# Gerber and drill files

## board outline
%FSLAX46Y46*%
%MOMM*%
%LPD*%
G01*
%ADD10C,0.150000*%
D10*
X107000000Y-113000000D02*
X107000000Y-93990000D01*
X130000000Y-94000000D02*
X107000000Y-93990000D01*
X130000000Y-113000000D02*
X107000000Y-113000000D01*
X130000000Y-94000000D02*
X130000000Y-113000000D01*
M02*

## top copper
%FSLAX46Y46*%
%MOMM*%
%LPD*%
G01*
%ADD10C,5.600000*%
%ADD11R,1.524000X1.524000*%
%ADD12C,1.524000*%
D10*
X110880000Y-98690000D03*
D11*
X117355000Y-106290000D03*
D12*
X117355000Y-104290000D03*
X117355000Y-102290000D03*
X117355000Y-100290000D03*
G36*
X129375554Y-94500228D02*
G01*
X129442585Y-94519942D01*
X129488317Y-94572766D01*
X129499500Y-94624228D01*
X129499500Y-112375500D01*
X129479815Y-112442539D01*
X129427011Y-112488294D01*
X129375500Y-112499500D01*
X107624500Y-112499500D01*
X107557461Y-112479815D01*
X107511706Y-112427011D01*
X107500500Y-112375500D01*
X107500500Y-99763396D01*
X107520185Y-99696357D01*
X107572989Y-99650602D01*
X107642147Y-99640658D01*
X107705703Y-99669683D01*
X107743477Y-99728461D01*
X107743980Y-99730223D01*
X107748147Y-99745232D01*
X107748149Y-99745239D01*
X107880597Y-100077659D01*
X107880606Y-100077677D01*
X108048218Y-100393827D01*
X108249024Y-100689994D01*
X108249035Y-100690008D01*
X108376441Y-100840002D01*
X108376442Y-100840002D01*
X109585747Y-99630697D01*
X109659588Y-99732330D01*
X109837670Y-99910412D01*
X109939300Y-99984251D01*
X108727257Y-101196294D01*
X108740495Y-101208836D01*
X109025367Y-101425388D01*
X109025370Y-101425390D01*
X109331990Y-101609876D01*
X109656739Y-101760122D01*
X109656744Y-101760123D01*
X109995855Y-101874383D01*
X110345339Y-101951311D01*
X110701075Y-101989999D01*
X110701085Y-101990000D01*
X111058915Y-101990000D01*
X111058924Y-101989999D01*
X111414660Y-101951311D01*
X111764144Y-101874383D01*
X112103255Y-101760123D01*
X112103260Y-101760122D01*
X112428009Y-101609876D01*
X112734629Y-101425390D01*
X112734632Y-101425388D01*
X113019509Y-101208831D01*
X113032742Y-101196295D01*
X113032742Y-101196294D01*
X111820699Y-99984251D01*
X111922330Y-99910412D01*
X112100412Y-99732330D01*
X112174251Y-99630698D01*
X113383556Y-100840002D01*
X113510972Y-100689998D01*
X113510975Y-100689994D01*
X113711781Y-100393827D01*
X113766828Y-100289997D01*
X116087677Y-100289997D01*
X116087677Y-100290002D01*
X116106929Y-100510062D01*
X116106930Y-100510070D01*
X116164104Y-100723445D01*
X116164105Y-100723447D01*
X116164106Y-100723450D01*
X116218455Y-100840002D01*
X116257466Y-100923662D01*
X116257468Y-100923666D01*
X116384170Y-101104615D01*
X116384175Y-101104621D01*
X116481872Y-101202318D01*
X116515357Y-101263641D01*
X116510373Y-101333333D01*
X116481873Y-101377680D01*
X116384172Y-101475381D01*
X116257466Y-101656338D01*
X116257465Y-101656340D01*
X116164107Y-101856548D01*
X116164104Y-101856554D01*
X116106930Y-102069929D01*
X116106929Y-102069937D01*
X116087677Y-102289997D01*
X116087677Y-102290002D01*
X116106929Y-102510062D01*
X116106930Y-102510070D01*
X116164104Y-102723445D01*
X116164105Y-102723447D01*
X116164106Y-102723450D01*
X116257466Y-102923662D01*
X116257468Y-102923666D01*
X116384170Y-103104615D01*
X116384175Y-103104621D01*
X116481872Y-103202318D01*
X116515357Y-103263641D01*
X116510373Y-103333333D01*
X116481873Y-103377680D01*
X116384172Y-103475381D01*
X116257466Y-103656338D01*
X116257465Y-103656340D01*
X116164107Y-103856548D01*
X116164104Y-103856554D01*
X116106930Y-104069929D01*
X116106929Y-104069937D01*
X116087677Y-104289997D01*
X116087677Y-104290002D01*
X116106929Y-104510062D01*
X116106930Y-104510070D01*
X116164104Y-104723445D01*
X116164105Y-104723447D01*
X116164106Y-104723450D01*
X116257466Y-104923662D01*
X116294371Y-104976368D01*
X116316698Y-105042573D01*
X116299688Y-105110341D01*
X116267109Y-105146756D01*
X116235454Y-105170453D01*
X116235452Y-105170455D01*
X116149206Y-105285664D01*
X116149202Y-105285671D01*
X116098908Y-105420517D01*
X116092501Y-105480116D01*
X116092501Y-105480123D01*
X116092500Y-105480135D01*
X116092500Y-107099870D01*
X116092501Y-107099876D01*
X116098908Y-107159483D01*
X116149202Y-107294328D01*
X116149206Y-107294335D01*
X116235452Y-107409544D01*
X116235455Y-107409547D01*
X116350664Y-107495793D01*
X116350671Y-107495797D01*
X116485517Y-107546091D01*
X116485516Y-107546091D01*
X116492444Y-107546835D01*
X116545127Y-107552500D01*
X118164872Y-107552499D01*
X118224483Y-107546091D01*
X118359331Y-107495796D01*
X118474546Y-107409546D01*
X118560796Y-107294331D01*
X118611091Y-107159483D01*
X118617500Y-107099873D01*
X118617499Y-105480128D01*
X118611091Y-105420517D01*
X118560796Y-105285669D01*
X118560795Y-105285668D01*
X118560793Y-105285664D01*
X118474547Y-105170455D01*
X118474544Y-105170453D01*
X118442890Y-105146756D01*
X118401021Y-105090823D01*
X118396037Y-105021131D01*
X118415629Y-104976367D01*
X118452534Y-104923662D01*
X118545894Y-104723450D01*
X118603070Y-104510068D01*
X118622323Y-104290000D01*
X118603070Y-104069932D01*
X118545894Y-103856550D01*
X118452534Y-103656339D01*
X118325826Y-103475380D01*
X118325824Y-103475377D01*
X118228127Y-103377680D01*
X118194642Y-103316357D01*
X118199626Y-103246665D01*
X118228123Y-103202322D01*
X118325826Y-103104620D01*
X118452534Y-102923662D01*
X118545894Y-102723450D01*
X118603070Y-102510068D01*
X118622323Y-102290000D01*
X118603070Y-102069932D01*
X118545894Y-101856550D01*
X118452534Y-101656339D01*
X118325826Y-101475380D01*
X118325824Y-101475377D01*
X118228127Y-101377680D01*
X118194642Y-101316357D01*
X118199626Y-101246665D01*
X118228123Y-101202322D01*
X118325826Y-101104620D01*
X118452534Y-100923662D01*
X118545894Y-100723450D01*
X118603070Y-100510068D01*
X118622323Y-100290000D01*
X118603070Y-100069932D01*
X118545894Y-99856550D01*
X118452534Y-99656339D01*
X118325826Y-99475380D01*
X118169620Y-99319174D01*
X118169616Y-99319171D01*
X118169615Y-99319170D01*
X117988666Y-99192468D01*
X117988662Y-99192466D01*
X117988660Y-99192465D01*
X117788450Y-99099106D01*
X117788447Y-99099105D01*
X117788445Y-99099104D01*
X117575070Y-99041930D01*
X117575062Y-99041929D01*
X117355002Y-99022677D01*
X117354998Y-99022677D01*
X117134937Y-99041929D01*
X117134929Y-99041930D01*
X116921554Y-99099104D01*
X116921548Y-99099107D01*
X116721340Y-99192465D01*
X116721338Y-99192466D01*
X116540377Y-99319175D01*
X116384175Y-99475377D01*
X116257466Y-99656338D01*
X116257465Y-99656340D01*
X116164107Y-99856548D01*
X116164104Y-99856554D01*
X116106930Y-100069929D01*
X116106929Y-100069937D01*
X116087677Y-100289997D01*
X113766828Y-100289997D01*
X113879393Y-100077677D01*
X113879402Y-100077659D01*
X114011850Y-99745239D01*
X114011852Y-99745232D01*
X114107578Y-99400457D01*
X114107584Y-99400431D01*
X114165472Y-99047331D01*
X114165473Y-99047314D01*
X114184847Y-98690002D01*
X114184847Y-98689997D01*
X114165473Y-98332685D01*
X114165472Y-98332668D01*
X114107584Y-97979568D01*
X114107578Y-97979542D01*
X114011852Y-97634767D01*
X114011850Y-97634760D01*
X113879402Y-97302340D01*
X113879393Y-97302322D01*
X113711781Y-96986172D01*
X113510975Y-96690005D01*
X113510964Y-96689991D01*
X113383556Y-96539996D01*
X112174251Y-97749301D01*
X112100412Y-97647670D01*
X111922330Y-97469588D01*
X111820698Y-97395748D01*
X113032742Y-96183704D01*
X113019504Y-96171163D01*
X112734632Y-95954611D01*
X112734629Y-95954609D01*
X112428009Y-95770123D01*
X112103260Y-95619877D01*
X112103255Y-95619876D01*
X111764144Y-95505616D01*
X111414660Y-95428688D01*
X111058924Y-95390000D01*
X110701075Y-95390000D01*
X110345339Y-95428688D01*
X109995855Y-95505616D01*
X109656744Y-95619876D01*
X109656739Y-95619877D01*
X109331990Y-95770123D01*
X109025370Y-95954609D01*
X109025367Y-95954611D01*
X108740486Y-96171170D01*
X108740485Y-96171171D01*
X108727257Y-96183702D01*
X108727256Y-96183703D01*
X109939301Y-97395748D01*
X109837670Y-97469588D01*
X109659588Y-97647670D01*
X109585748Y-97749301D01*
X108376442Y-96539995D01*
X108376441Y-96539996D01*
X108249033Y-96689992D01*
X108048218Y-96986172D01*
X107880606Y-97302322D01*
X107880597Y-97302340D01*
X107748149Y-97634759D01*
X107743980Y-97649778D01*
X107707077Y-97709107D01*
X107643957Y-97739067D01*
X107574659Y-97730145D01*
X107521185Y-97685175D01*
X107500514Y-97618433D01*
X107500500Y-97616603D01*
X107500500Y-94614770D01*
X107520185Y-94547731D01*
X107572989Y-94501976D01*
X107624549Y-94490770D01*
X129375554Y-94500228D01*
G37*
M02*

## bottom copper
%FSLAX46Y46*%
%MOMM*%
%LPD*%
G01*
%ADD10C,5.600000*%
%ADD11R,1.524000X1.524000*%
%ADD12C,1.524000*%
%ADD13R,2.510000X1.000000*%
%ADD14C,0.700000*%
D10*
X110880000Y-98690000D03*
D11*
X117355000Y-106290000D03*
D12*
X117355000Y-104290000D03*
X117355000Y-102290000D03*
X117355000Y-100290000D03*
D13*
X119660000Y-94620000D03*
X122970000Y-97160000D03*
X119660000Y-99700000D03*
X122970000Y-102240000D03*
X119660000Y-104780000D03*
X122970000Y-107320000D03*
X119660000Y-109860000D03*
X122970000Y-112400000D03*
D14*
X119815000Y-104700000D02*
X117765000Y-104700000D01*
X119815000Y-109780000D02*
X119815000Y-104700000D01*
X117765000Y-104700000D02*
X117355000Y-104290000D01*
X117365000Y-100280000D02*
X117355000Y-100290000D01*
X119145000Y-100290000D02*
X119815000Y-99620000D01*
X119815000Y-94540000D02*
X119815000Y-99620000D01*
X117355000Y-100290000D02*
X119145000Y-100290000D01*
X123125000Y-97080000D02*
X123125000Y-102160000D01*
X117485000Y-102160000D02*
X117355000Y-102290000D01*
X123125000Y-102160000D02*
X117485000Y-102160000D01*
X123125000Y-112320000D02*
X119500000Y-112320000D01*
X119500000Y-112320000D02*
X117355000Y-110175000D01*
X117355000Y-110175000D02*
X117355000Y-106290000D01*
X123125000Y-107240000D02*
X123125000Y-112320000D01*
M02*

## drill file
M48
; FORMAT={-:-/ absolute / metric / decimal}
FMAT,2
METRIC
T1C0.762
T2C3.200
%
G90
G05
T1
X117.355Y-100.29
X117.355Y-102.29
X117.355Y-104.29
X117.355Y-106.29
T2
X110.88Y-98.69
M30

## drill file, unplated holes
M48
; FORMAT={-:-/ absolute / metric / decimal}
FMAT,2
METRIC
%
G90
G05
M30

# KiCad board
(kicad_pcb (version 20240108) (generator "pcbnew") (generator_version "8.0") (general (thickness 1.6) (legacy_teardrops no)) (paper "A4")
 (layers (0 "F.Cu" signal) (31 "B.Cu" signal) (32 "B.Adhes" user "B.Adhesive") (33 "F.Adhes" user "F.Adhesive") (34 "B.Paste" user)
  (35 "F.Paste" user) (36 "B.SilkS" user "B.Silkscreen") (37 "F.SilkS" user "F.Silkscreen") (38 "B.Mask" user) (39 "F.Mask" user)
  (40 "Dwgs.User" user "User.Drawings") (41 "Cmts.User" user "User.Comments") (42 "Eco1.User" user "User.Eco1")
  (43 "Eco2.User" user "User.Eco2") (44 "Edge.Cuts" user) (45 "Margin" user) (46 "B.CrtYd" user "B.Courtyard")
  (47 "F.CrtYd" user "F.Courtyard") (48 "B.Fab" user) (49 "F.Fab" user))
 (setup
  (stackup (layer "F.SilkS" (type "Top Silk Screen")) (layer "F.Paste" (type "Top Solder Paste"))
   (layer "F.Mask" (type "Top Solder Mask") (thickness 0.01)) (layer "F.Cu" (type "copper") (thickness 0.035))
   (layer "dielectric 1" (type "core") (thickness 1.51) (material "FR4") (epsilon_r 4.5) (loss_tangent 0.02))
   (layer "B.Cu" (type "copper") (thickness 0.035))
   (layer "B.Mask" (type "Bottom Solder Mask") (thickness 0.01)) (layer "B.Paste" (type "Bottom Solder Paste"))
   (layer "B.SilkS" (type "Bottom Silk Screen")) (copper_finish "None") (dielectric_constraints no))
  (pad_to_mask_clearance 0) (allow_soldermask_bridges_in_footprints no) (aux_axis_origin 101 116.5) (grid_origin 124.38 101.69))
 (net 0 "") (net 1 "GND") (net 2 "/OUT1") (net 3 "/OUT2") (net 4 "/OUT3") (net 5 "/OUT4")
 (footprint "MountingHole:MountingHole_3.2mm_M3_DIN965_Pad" (layer "F.Cu") (at 110.88 98.69)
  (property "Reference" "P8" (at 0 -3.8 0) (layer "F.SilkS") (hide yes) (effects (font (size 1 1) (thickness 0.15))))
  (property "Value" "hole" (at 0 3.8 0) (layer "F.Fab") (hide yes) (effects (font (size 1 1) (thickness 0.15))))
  (pad "1" thru_hole circle (at 0 0) (size 5.6 5.6) (drill 3.2) (layers "*.Cu" "*.Mask") (remove_unused_layers no) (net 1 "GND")))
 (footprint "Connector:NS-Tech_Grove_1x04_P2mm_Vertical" (layer "F.Cu") (at 117.355 106.29 180)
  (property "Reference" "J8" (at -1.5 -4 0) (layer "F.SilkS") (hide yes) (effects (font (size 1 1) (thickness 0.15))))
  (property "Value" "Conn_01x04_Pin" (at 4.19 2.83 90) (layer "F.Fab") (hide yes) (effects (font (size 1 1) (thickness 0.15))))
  (pad "1" thru_hole rect (at 0 0 180) (size 1.524 1.524) (drill 0.762) (layers "*.Cu" "*.Mask") (remove_unused_layers no) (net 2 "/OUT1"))
  (pad "2" thru_hole circle (at 0 2 180) (size 1.524 1.524) (drill 0.762) (layers "*.Cu" "*.Mask") (remove_unused_layers no) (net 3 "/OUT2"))
  (pad "3" thru_hole circle (at 0 4 180) (size 1.524 1.524) (drill 0.762) (layers "*.Cu" "*.Mask") (remove_unused_layers no) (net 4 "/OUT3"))
  (pad "4" thru_hole circle (at 0 6 180) (size 1.524 1.524) (drill 0.762) (layers "*.Cu" "*.Mask") (remove_unused_layers no) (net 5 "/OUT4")))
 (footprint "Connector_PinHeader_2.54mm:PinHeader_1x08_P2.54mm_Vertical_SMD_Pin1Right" (layer "B.Cu") (at 121.315 103.51 180)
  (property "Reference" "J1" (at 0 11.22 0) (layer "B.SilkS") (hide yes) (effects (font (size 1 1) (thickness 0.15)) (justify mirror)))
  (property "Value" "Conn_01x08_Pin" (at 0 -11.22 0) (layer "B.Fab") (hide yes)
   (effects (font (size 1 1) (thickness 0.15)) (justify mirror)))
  (pad "1" smd rect (at 1.655 8.89 180) (size 2.51 1) (layers "B.Cu" "B.Paste" "B.Mask") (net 5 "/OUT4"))
  (pad "2" smd rect (at -1.655 6.35 180) (size 2.51 1) (layers "B.Cu" "B.Paste" "B.Mask") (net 4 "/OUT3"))
  (pad "3" smd rect (at 1.655 3.81 180) (size 2.51 1) (layers "B.Cu" "B.Paste" "B.Mask") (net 5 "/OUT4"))
  (pad "4" smd rect (at -1.655 1.27 180) (size 2.51 1) (layers "B.Cu" "B.Paste" "B.Mask") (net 4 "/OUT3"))
  (pad "5" smd rect (at 1.655 -1.27 180) (size 2.51 1) (layers "B.Cu" "B.Paste" "B.Mask") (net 3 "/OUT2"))
  (pad "6" smd rect (at -1.655 -3.81 180) (size 2.51 1) (layers "B.Cu" "B.Paste" "B.Mask") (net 2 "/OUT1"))
  (pad "7" smd rect (at 1.655 -6.35 180) (size 2.51 1) (layers "B.Cu" "B.Paste" "B.Mask") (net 3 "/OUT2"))
  (pad "8" smd rect (at -1.655 -8.89 180) (size 2.51 1) (layers "B.Cu" "B.Paste" "B.Mask") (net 2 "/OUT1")))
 (gr_line (start 107 113) (end 107 93.99) (stroke (width 0.15) (type solid)) (layer "Edge.Cuts"))
 (gr_line (start 130 94) (end 107 93.99) (stroke (width 0.15) (type solid)) (layer "Edge.Cuts"))
 (gr_line (start 130 113) (end 107 113) (stroke (width 0.15) (type solid)) (layer "Edge.Cuts"))
 (gr_line (start 130 94) (end 130 113) (stroke (width 0.15) (type solid)) (layer "Edge.Cuts"))
 (segment (start 119.815 104.7) (end 117.765 104.7) (width 0.7) (layer "B.Cu") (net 3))
 (segment (start 119.815 109.78) (end 119.815 104.7) (width 0.7) (layer "B.Cu") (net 3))
 (segment (start 117.765 104.7) (end 117.355 104.29) (width 0.7) (layer "B.Cu") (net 3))
 (segment (start 117.365 100.28) (end 117.355 100.29) (width 0.7) (layer "B.Cu") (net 5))
 (segment (start 119.145 100.29) (end 119.815 99.62) (width 0.7) (layer "B.Cu") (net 5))
 (segment (start 119.815 94.54) (end 119.815 99.62) (width 0.7) (layer "B.Cu") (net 5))
 (segment (start 117.355 100.29) (end 119.145 100.29) (width 0.7) (layer "B.Cu") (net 5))
 (segment (start 123.125 97.08) (end 123.125 102.16) (width 0.7) (layer "B.Cu") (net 4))
 (segment (start 117.485 102.16) (end 117.355 102.29) (width 0.7) (layer "B.Cu") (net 4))
 (segment (start 123.125 102.16) (end 117.485 102.16) (width 0.7) (layer "B.Cu") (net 4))
 (segment (start 123.125 112.32) (end 119.5 112.32) (width 0.7) (layer "B.Cu") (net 2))
 (segment (start 119.5 112.32) (end 117.355 110.175) (width 0.7) (layer "B.Cu") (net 2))
 (segment (start 117.355 110.175) (end 117.355 106.29) (width 0.7) (layer "B.Cu") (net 2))
 (segment (start 123.125 107.24) (end 123.125 112.32) (width 0.7) (layer "B.Cu") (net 2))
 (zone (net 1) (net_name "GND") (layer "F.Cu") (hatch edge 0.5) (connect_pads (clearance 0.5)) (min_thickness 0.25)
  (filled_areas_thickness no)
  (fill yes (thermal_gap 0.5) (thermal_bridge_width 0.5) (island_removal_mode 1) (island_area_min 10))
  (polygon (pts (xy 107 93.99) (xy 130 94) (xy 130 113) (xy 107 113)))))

